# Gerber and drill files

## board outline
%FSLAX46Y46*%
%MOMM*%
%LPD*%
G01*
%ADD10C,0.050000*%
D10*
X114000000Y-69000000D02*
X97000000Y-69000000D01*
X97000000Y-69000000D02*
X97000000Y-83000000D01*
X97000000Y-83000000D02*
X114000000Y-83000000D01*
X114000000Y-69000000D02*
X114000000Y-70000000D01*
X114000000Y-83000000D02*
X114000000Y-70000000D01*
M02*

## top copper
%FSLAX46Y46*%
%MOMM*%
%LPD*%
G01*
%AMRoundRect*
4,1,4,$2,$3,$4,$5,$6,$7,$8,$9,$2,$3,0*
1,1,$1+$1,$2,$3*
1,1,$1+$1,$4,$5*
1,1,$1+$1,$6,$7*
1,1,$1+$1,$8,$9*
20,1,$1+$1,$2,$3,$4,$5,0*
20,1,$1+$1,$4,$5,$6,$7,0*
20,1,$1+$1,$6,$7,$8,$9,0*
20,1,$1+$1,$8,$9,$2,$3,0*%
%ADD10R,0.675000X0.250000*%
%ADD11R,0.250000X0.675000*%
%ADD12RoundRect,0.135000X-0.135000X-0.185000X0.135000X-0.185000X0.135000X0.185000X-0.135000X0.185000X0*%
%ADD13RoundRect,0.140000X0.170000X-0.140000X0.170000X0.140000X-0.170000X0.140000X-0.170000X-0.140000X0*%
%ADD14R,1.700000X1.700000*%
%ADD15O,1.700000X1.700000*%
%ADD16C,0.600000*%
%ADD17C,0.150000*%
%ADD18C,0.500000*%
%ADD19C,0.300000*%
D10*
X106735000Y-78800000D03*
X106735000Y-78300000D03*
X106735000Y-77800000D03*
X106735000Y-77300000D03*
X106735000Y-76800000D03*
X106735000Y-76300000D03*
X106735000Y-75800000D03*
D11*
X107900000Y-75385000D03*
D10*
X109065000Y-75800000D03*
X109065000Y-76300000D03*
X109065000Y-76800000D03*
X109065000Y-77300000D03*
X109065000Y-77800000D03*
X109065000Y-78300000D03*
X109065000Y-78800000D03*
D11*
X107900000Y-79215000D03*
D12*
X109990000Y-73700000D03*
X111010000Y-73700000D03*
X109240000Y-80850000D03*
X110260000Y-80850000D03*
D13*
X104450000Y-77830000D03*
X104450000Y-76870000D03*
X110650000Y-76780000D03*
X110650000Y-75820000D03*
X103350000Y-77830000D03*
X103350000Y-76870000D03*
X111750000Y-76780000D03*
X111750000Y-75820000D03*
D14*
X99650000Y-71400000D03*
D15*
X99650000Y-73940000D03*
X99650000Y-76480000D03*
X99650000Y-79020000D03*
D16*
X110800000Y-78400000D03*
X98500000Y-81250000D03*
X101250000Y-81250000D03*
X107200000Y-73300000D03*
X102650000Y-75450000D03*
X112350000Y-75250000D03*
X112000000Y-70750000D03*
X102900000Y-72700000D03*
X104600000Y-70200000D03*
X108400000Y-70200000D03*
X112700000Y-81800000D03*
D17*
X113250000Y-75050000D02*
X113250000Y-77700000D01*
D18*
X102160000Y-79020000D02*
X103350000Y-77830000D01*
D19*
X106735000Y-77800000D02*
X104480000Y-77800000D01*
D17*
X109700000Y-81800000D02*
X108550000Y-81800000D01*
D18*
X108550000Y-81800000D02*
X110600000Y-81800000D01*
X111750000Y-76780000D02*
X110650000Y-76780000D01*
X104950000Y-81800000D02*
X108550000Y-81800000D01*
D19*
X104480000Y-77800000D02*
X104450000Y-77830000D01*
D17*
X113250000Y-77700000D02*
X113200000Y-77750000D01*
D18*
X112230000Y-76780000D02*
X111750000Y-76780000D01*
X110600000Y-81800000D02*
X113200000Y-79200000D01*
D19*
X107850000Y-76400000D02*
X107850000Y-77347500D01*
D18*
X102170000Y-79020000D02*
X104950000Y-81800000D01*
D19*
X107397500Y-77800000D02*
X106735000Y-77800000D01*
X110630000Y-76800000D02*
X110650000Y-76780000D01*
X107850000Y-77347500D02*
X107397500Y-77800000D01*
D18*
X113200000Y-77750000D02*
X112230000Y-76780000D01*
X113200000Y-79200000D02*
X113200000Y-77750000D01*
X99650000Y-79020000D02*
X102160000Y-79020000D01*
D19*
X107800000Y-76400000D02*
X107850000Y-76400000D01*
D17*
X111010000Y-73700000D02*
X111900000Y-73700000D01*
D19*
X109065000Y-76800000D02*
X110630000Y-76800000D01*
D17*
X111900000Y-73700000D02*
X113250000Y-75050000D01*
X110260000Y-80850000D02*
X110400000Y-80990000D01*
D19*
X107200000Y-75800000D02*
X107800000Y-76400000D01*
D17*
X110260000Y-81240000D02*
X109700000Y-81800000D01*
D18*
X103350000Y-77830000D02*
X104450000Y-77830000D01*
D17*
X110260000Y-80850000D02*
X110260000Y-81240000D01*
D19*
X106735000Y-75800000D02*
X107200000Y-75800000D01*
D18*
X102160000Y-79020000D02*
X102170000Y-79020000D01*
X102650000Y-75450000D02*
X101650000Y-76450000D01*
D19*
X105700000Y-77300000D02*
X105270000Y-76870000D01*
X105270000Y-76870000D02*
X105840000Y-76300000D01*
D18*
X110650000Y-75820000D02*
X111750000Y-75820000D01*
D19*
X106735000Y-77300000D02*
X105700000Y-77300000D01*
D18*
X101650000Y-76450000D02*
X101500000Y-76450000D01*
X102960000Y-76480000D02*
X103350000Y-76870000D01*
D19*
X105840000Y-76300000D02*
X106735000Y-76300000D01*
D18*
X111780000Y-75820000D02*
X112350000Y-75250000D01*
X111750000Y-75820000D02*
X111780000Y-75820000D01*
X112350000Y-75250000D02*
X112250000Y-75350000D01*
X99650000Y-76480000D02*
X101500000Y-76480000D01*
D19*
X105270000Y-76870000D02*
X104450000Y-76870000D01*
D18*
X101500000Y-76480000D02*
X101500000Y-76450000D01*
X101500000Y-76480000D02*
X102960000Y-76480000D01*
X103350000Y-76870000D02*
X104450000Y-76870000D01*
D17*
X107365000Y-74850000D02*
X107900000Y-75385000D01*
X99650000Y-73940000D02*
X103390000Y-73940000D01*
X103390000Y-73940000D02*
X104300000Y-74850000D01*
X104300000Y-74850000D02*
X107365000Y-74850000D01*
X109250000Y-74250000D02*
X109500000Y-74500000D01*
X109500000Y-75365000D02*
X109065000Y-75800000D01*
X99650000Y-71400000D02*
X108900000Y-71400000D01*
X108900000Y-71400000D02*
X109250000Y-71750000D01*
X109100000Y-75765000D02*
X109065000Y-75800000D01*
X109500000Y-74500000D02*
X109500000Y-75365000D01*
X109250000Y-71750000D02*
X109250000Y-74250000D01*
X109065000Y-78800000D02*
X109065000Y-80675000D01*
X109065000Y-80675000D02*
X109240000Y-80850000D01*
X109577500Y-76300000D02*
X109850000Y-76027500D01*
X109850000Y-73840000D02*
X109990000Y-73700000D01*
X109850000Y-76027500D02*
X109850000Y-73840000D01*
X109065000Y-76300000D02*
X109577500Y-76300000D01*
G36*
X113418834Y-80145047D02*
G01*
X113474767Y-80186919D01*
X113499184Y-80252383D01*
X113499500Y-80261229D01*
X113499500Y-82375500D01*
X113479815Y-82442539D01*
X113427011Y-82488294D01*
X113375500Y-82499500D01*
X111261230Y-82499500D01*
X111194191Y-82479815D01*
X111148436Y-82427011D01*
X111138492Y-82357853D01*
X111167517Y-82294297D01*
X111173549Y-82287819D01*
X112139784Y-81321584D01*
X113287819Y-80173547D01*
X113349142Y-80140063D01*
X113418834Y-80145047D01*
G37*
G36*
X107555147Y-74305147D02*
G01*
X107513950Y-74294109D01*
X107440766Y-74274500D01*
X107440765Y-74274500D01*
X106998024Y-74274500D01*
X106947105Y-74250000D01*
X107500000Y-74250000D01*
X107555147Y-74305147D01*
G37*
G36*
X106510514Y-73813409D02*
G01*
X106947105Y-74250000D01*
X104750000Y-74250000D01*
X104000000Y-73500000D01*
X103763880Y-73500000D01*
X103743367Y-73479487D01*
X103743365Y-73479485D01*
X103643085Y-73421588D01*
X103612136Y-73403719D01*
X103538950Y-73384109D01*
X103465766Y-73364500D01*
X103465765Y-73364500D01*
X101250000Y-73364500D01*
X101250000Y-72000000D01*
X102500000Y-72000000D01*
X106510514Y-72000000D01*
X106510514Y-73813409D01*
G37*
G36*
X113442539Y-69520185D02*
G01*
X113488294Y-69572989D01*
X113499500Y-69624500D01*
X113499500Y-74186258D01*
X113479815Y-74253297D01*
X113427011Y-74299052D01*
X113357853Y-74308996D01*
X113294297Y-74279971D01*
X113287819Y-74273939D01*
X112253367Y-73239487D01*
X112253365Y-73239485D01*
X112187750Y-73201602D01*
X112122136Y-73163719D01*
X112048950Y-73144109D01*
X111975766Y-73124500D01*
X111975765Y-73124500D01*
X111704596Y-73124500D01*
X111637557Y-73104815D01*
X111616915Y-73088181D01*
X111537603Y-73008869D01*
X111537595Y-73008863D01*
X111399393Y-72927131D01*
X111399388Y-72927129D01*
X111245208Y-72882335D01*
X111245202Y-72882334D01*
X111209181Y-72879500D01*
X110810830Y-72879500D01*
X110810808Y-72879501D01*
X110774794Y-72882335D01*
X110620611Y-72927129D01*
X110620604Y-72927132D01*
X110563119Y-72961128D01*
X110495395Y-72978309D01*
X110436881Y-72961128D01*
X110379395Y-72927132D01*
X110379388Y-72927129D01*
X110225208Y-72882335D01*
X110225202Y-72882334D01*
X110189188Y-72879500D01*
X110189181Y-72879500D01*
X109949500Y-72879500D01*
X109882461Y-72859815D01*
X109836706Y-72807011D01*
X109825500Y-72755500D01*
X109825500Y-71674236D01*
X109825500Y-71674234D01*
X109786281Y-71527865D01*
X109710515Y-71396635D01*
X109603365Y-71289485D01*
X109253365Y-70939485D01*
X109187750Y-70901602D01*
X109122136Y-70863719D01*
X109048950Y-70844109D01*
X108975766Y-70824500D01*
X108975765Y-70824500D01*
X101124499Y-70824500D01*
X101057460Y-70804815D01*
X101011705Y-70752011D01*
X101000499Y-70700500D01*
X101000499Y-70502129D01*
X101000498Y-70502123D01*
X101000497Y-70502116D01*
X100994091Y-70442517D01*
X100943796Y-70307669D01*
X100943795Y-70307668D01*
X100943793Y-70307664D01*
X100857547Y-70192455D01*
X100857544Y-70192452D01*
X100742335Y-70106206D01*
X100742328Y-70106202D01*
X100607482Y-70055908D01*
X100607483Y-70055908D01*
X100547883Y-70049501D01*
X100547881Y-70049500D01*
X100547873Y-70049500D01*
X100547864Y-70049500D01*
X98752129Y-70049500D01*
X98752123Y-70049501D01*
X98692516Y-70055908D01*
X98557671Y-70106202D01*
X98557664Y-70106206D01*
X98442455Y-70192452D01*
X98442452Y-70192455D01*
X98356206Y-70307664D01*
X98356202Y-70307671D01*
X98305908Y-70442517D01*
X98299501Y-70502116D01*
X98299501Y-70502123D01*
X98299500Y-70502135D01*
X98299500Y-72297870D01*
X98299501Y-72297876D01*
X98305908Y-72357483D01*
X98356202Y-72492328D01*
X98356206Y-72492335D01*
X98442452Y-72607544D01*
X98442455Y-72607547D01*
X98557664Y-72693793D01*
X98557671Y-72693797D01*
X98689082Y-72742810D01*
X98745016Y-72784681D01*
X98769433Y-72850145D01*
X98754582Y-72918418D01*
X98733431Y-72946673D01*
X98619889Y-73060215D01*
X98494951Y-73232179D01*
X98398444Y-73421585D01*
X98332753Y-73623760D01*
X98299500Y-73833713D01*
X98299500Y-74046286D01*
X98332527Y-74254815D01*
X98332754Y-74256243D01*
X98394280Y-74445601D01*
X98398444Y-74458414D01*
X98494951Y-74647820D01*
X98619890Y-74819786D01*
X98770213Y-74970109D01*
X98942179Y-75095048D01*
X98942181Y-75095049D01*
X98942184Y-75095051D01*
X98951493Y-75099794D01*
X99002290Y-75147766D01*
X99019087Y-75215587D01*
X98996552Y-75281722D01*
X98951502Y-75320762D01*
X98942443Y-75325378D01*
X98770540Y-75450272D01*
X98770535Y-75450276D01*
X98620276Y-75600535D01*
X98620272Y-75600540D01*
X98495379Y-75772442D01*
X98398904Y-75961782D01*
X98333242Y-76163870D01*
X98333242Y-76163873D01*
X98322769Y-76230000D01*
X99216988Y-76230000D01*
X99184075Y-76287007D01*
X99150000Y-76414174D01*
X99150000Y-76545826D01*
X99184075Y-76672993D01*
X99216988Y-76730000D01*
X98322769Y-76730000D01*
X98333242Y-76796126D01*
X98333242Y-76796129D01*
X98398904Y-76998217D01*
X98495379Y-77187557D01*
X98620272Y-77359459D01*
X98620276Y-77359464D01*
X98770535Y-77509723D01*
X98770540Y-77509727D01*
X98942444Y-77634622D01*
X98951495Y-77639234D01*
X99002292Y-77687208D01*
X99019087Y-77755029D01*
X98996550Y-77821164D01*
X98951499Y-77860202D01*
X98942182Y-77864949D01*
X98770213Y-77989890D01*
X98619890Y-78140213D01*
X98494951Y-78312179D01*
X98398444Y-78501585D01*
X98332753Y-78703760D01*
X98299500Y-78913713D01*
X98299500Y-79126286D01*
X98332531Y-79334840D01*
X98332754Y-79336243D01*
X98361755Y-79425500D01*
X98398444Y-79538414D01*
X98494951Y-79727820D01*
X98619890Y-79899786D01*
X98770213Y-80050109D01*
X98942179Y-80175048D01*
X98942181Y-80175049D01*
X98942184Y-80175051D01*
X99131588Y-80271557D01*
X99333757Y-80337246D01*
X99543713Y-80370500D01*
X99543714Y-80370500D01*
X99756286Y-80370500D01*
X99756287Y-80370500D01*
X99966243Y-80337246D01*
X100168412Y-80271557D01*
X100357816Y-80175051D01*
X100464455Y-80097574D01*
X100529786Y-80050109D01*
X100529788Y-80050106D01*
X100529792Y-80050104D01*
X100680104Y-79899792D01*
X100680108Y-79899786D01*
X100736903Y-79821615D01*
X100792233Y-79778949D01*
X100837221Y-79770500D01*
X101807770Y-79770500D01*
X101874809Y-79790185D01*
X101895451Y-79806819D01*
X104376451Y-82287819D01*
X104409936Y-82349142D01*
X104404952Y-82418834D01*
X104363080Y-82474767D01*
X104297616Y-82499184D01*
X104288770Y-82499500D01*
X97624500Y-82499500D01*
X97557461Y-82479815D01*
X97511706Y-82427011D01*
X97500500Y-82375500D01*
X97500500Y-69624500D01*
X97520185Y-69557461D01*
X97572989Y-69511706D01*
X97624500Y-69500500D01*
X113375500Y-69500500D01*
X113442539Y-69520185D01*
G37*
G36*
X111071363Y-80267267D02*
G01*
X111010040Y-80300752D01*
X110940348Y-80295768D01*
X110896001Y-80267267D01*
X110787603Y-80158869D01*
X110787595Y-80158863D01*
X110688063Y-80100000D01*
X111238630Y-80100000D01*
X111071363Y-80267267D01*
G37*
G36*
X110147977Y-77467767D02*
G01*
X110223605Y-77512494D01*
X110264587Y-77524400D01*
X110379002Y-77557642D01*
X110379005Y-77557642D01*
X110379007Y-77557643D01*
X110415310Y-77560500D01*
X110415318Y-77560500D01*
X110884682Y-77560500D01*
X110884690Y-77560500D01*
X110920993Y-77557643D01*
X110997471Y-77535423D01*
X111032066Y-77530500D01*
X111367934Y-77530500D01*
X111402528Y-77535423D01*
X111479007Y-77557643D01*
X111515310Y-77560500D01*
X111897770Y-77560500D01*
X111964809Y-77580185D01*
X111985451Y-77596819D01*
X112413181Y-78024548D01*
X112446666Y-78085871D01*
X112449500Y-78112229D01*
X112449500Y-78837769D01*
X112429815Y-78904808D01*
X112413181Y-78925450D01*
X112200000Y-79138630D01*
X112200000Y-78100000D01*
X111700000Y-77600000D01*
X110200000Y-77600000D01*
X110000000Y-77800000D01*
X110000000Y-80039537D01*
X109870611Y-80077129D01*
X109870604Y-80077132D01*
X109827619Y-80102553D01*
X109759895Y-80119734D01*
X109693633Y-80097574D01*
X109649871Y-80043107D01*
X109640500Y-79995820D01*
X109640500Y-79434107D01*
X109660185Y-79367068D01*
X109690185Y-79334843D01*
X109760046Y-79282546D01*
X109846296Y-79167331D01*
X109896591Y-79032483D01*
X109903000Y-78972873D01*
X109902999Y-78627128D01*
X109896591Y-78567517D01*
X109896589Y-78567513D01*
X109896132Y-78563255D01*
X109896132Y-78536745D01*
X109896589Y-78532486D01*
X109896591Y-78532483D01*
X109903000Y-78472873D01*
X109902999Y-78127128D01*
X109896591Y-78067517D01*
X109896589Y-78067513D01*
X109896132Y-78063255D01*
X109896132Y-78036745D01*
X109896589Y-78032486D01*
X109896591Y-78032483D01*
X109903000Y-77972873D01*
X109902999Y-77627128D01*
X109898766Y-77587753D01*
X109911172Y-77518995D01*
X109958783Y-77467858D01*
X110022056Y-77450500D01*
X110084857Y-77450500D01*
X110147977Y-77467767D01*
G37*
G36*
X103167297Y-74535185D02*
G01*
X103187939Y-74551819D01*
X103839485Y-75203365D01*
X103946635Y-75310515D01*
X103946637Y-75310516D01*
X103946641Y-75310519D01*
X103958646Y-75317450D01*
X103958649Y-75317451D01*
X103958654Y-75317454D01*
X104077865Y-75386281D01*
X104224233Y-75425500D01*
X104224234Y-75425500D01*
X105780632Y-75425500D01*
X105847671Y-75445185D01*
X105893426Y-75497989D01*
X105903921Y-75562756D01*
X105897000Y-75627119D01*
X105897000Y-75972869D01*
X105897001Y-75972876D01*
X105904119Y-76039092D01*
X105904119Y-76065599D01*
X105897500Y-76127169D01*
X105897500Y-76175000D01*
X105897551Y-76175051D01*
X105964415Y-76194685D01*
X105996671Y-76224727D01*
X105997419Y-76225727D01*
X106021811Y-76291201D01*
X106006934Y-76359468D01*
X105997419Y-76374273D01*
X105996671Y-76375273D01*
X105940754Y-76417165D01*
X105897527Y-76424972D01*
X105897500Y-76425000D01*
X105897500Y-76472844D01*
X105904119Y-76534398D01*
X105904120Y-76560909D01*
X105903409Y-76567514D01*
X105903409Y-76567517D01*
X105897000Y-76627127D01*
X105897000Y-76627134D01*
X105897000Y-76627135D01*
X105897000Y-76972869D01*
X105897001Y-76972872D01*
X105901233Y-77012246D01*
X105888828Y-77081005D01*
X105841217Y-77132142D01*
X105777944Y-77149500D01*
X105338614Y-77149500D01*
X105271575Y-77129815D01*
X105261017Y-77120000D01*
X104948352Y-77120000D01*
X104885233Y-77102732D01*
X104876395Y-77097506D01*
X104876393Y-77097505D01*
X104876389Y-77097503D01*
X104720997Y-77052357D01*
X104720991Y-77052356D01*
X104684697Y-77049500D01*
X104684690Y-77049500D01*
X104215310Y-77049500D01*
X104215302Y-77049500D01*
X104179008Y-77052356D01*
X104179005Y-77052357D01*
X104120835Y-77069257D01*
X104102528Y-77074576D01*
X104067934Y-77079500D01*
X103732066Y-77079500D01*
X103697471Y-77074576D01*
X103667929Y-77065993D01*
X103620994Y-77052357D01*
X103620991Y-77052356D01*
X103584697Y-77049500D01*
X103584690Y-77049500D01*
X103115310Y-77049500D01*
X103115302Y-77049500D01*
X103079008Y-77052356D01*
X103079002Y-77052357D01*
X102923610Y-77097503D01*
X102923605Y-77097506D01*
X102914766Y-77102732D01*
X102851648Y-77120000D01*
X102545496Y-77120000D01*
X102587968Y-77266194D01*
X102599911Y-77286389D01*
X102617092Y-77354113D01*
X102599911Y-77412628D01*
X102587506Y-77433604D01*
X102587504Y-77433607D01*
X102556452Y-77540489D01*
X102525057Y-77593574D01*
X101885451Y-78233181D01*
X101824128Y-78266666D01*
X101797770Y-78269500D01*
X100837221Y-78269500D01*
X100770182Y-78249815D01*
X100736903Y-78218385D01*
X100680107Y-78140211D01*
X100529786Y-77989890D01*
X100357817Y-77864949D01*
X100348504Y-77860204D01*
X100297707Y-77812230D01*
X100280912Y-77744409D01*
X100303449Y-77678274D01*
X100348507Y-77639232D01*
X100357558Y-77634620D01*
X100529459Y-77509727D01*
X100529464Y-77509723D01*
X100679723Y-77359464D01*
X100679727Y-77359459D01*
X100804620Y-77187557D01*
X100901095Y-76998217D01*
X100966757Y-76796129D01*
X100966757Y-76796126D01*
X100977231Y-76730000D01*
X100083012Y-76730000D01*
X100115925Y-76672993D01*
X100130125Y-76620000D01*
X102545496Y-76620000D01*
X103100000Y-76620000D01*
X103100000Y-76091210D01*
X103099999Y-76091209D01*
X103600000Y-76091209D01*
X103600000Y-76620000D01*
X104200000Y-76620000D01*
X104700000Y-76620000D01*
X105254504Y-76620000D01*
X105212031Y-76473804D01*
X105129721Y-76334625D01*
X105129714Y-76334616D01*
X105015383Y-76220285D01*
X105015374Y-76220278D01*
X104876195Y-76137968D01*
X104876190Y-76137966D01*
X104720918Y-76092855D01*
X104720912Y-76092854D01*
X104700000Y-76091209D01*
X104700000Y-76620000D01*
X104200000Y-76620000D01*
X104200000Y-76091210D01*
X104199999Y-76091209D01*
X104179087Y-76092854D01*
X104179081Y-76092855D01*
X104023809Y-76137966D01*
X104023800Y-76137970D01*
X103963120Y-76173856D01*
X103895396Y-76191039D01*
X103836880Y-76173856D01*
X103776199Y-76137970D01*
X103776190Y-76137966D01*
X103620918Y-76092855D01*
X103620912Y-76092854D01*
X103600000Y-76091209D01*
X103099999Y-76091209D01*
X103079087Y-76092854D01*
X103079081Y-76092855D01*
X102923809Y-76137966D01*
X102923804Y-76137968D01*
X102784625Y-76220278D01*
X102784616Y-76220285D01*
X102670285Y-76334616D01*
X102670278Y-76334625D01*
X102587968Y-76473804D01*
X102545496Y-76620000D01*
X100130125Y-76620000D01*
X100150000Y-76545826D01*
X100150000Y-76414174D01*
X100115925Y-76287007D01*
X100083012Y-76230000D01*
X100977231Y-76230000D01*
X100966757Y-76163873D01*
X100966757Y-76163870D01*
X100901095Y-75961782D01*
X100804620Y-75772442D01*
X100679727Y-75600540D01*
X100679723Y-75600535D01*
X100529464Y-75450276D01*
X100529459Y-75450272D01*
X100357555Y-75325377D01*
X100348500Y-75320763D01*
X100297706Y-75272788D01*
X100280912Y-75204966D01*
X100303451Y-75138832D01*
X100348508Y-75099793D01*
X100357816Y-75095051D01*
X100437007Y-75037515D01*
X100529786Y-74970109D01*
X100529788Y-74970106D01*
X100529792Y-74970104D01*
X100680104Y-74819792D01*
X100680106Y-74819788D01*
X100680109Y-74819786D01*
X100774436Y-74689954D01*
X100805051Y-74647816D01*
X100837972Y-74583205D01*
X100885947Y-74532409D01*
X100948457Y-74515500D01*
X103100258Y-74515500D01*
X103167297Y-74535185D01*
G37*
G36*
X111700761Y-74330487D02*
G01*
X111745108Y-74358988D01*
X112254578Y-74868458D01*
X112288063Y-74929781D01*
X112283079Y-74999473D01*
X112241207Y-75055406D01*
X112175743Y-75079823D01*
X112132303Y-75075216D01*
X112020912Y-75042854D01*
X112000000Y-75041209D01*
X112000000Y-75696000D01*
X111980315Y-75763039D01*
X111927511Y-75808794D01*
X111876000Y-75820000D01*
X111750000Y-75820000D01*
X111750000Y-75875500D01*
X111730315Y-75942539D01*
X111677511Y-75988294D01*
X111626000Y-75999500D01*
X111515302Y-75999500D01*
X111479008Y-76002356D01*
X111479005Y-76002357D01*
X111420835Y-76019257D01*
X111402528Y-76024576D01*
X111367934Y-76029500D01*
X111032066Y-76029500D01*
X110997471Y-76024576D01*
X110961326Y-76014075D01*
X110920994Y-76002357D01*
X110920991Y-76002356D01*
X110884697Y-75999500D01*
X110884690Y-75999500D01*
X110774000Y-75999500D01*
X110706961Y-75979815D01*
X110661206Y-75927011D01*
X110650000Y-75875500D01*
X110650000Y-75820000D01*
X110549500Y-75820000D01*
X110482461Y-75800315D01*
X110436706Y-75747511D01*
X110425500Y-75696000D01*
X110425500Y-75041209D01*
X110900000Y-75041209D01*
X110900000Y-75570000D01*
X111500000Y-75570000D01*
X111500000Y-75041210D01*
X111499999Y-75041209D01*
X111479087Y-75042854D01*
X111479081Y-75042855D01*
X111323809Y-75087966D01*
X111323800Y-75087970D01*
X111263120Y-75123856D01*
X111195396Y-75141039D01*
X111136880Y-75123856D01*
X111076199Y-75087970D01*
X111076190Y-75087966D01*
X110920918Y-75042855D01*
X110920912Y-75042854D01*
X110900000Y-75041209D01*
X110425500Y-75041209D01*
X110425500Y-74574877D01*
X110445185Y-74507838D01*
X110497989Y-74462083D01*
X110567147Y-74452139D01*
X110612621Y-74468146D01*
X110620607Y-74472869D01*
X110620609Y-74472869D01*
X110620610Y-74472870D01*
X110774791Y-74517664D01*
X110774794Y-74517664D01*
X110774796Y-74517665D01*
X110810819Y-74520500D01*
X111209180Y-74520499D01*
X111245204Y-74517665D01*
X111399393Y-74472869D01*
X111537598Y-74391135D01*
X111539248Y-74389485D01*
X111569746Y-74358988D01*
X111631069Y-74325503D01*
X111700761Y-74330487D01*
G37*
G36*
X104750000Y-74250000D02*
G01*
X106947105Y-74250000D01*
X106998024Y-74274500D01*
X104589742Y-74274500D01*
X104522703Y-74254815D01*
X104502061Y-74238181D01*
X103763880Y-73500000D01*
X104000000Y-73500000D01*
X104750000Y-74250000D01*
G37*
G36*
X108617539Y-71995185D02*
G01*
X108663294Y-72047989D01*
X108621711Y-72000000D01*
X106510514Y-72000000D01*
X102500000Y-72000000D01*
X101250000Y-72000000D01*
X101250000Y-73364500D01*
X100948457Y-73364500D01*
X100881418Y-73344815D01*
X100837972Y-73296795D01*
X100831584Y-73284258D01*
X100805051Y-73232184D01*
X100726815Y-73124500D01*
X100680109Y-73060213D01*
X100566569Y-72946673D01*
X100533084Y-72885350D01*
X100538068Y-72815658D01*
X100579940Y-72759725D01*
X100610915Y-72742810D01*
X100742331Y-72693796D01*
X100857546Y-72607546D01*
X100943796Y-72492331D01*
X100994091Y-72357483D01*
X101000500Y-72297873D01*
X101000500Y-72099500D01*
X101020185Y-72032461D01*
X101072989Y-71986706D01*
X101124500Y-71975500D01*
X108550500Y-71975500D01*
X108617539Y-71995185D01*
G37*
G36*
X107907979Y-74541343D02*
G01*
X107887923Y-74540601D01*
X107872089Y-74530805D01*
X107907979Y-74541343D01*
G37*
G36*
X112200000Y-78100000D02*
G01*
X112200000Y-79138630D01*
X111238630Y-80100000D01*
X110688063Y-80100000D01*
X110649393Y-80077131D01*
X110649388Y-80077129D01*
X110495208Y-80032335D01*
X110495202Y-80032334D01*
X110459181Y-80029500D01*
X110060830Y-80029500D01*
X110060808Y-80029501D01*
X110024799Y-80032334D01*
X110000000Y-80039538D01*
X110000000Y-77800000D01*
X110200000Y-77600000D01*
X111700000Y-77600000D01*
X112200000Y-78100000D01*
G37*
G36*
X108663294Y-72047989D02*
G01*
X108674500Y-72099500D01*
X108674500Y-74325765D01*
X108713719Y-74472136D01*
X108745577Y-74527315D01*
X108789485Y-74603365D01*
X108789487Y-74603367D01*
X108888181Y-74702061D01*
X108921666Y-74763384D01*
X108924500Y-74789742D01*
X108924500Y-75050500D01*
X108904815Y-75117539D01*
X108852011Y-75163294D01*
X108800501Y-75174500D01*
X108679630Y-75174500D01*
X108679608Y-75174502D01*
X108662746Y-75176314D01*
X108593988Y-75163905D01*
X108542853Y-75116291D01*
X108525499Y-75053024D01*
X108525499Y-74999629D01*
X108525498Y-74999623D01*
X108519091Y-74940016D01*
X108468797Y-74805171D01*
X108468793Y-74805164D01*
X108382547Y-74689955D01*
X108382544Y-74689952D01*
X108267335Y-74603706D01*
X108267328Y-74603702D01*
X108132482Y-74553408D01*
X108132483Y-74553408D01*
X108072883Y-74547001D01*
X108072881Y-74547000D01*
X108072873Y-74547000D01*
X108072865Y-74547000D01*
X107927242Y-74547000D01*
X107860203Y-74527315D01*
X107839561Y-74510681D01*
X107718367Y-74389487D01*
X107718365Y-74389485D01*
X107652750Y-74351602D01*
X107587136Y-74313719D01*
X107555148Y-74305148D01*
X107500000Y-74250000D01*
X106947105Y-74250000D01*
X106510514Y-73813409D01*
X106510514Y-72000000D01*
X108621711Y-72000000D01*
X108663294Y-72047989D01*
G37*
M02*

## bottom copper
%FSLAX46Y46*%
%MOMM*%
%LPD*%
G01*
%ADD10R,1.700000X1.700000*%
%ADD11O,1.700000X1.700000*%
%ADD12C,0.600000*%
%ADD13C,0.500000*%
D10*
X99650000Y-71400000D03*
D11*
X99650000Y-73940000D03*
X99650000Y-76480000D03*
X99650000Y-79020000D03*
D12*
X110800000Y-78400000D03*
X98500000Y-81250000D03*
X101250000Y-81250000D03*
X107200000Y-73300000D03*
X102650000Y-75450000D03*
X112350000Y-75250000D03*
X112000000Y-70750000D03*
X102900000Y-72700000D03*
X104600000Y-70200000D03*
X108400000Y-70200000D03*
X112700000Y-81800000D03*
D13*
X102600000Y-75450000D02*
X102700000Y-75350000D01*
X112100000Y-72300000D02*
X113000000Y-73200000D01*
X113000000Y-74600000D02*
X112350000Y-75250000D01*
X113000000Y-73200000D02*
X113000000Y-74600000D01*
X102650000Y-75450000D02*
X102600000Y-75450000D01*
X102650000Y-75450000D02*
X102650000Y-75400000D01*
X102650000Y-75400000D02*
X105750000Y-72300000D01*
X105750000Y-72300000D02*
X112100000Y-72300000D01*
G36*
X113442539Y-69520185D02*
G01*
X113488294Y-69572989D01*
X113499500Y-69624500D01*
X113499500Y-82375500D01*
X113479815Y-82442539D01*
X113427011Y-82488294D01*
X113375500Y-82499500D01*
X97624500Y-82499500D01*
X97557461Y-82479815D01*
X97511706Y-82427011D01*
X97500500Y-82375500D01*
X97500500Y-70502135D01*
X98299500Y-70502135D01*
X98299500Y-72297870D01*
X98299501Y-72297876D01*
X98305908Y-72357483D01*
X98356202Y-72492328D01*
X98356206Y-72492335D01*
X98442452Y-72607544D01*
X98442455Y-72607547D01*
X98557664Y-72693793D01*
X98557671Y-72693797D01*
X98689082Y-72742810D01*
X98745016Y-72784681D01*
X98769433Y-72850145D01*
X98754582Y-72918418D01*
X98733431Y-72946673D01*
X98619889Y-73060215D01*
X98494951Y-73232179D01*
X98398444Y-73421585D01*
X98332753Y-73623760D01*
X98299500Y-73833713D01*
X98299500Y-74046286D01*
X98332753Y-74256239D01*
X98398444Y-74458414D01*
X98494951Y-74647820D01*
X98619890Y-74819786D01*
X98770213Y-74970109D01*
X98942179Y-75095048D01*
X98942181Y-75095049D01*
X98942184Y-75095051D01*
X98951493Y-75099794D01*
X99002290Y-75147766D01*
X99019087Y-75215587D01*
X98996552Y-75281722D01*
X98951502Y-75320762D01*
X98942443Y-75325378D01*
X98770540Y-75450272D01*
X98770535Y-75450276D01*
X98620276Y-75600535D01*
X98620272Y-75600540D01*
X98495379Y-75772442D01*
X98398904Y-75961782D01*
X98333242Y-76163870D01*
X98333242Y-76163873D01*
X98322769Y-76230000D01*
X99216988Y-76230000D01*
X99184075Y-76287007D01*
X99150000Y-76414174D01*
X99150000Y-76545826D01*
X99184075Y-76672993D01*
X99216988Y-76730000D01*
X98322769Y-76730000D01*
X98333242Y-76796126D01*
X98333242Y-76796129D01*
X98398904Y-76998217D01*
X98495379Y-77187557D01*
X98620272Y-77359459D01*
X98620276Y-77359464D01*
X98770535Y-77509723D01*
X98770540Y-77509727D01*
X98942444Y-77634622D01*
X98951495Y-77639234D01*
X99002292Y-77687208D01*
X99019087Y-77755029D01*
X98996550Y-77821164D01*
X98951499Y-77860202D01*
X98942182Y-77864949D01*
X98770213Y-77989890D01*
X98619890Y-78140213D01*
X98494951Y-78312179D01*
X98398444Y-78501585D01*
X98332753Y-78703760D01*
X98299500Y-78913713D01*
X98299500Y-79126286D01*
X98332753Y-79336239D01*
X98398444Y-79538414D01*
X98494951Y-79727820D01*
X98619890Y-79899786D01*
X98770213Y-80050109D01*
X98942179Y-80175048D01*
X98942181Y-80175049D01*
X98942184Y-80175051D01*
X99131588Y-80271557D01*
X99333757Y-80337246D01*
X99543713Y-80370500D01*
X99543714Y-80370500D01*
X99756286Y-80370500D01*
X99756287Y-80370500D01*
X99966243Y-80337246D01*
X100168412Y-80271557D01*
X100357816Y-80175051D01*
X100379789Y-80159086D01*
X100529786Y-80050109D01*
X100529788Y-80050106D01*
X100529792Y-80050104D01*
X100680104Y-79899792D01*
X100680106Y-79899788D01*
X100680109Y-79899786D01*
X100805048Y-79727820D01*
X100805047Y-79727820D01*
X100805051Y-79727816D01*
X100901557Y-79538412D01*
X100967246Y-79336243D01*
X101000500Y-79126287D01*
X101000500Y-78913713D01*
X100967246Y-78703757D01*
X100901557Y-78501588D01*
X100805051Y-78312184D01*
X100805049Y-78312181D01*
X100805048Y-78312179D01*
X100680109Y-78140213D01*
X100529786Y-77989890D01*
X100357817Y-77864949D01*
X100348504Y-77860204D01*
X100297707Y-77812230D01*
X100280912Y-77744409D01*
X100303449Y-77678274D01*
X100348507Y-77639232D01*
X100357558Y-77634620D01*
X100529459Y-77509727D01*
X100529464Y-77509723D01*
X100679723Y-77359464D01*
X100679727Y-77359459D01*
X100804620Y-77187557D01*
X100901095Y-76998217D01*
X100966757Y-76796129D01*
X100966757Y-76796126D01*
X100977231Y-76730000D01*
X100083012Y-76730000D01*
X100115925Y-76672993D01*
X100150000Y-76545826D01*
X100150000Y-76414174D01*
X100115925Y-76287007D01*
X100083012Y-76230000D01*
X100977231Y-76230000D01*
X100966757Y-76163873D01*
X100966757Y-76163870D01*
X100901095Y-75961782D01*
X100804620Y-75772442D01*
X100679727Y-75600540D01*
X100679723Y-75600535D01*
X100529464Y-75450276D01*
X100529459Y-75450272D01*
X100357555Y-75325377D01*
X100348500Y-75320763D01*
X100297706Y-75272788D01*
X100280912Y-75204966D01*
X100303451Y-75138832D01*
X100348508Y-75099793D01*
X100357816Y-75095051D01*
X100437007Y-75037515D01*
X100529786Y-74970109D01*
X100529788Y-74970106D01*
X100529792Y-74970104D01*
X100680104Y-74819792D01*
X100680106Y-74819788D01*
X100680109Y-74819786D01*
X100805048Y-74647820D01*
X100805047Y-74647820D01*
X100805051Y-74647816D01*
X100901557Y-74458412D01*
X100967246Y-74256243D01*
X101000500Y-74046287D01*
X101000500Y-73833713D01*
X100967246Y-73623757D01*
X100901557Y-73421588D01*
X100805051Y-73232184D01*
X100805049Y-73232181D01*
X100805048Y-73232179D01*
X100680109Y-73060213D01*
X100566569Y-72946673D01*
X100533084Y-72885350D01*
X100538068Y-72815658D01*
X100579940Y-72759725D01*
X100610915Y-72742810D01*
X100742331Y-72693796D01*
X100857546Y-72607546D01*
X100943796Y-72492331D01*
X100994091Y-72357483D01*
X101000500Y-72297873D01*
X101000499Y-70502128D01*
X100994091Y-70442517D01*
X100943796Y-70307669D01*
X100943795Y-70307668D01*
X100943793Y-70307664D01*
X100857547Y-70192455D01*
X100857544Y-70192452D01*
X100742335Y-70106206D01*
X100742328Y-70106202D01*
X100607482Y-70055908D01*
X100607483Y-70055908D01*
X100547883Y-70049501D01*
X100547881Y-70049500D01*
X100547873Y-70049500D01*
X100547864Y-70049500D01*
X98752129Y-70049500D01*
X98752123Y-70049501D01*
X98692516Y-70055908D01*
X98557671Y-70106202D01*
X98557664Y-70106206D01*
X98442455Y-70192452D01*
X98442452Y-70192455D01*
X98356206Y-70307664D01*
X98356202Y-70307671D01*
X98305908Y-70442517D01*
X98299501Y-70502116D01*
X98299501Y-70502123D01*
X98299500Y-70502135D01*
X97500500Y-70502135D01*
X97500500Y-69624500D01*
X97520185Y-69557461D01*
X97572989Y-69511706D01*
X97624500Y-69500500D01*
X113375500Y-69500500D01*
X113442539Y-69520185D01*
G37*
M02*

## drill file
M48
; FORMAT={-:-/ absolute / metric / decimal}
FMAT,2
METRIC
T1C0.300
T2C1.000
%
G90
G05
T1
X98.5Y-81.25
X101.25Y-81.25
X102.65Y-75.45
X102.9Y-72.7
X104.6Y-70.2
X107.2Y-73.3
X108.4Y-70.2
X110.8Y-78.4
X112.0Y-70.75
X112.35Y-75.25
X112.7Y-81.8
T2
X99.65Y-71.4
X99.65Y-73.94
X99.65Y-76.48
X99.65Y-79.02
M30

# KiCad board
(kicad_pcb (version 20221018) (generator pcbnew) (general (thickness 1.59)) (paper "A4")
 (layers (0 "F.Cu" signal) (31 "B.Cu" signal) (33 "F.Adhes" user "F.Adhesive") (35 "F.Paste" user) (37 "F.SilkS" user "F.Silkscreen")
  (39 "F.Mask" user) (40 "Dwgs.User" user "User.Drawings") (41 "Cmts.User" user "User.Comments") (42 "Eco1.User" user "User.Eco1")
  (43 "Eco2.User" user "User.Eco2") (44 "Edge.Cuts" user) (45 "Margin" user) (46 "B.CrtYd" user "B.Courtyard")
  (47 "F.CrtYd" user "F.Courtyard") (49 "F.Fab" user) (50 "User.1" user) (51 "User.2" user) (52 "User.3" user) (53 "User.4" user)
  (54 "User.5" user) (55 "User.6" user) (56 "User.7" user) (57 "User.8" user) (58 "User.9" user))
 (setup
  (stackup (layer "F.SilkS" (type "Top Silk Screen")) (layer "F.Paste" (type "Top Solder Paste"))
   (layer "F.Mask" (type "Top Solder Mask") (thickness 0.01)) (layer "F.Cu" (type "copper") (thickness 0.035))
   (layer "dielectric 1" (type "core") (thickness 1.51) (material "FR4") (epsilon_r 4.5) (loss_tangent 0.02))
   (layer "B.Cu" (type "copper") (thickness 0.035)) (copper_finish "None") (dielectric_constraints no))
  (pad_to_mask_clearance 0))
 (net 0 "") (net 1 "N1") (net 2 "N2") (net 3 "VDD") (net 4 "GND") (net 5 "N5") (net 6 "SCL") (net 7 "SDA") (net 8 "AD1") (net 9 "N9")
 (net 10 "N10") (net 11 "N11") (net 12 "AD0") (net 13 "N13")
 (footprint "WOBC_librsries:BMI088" (layer "F.Cu") (at 107.9 77.3 90)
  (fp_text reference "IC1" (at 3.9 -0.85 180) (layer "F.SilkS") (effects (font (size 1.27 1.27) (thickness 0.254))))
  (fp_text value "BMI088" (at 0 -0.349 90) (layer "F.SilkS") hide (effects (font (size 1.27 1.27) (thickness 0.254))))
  (pad "1" smd rect (at -1.5 -1.165 90) (size 0.25 0.675) (layers "F.Cu" "F.Paste" "F.Mask") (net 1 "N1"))
  (pad "2" smd rect (at -1 -1.165 90) (size 0.25 0.675) (layers "F.Cu" "F.Paste" "F.Mask") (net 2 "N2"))
  (pad "3" smd rect (at -0.5 -1.165 90) (size 0.25 0.675) (layers "F.Cu" "F.Paste" "F.Mask") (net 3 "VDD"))
  (pad "4" smd rect (at 0 -1.165 90) (size 0.25 0.675) (layers "F.Cu" "F.Paste" "F.Mask") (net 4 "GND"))
  (pad "5" smd rect (at 0.5 -1.165 90) (size 0.25 0.675) (layers "F.Cu" "F.Paste" "F.Mask") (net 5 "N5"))
  (pad "6" smd rect (at 1 -1.165 90) (size 0.25 0.675) (layers "F.Cu" "F.Paste" "F.Mask") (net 4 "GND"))
  (pad "7" smd rect (at 1.5 -1.165 90) (size 0.25 0.675) (layers "F.Cu" "F.Paste" "F.Mask") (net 3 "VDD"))
  (pad "8" smd rect (at 1.915 0 180) (size 0.25 0.675) (layers "F.Cu" "F.Paste" "F.Mask") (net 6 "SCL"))
  (pad "9" smd rect (at 1.5 1.165 90) (size 0.25 0.675) (layers "F.Cu" "F.Paste" "F.Mask") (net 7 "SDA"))
  (pad "10" smd rect (at 1 1.165 90) (size 0.25 0.675) (layers "F.Cu" "F.Paste" "F.Mask") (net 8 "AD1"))
  (pad "11" smd rect (at 0.5 1.165 90) (size 0.25 0.675) (layers "F.Cu" "F.Paste" "F.Mask") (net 3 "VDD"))
  (pad "12" smd rect (at 0 1.165 90) (size 0.25 0.675) (layers "F.Cu" "F.Paste" "F.Mask") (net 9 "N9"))
  (pad "13" smd rect (at -0.5 1.165 90) (size 0.25 0.675) (layers "F.Cu" "F.Paste" "F.Mask") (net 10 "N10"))
  (pad "14" smd rect (at -1 1.165 90) (size 0.25 0.675) (layers "F.Cu" "F.Paste" "F.Mask") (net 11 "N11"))
  (pad "15" smd rect (at -1.5 1.165 90) (size 0.25 0.675) (layers "F.Cu" "F.Paste" "F.Mask") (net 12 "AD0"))
  (pad "16" smd rect (at -1.915 0 180) (size 0.25 0.675) (layers "F.Cu" "F.Paste" "F.Mask") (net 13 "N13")))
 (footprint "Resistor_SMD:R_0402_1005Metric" (layer "F.Cu") (at 110.5 73.7)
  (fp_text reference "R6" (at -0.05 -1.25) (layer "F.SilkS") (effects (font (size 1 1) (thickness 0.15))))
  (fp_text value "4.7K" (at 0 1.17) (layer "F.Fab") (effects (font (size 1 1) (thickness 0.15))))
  (pad "1" smd roundrect (at -0.51 0) (size 0.54 0.64) (layers "F.Cu" "F.Paste" "F.Mask") (roundrect_rratio 0.25) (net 8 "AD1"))
  (pad "2" smd roundrect (at 0.51 0) (size 0.54 0.64) (layers "F.Cu" "F.Paste" "F.Mask") (roundrect_rratio 0.25) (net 3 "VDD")))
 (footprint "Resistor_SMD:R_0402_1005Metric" (layer "F.Cu") (at 109.75 80.85)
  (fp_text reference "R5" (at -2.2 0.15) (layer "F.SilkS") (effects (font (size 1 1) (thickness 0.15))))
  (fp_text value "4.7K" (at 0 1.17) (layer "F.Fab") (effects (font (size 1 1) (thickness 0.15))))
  (pad "1" smd roundrect (at -0.51 0) (size 0.54 0.64) (layers "F.Cu" "F.Paste" "F.Mask") (roundrect_rratio 0.25) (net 12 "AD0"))
  (pad "2" smd roundrect (at 0.51 0) (size 0.54 0.64) (layers "F.Cu" "F.Paste" "F.Mask") (roundrect_rratio 0.25) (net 3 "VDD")))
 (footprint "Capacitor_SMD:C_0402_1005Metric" (layer "F.Cu") (at 104.45 77.35 90)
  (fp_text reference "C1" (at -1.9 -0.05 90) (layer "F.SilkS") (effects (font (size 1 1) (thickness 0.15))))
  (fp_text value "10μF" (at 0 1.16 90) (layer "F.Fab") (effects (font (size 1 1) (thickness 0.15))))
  (pad "1" smd roundrect (at -0.48 0 90) (size 0.56 0.62) (layers "F.Cu" "F.Paste" "F.Mask") (roundrect_rratio 0.25) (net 3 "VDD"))
  (pad "2" smd roundrect (at 0.48 0 90) (size 0.56 0.62) (layers "F.Cu" "F.Paste" "F.Mask") (roundrect_rratio 0.25) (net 4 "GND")))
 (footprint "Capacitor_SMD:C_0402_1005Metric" (layer "F.Cu") (at 110.65 76.3 90)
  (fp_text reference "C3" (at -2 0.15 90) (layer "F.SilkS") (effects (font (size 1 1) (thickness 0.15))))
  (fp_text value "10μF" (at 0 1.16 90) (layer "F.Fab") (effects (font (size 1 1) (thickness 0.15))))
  (pad "1" smd roundrect (at -0.48 0 90) (size 0.56 0.62) (layers "F.Cu" "F.Paste" "F.Mask") (roundrect_rratio 0.25) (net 3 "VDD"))
  (pad "2" smd roundrect (at 0.48 0 90) (size 0.56 0.62) (layers "F.Cu" "F.Paste" "F.Mask") (roundrect_rratio 0.25) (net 4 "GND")))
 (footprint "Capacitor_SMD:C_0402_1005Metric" (layer "F.Cu") (at 103.35 77.35 90)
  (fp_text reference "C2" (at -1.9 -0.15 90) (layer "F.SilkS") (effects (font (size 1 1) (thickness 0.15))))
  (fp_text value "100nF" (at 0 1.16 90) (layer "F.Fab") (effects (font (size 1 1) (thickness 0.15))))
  (pad "1" smd roundrect (at -0.48 0 90) (size 0.56 0.62) (layers "F.Cu" "F.Paste" "F.Mask") (roundrect_rratio 0.25) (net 3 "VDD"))
  (pad "2" smd roundrect (at 0.48 0 90) (size 0.56 0.62) (layers "F.Cu" "F.Paste" "F.Mask") (roundrect_rratio 0.25) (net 4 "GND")))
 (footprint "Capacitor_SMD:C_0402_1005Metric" (layer "F.Cu") (at 111.75 76.3 90)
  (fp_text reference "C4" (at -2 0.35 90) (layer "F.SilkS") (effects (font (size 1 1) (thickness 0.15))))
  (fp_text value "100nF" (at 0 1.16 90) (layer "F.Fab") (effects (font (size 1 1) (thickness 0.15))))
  (pad "1" smd roundrect (at -0.48 0 90) (size 0.56 0.62) (layers "F.Cu" "F.Paste" "F.Mask") (roundrect_rratio 0.25) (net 3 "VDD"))
  (pad "2" smd roundrect (at 0.48 0 90) (size 0.56 0.62) (layers "F.Cu" "F.Paste" "F.Mask") (roundrect_rratio 0.25) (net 4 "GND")))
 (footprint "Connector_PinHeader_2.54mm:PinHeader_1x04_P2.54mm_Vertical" (layer "F.Cu") (at 99.65 71.4)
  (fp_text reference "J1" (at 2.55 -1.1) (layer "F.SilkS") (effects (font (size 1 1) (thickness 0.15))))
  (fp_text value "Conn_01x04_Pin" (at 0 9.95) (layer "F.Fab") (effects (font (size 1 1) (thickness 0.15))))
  (pad "1" thru_hole rect (at 0 0) (size 1.7 1.7) (drill 1) (layers "*.Cu" "*.Mask") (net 7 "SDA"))
  (pad "2" thru_hole oval (at 0 2.54) (size 1.7 1.7) (drill 1) (layers "*.Cu" "*.Mask") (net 6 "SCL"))
  (pad "3" thru_hole oval (at 0 5.08) (size 1.7 1.7) (drill 1) (layers "*.Cu" "*.Mask") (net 4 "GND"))
  (pad "4" thru_hole oval (at 0 7.62) (size 1.7 1.7) (drill 1) (layers "*.Cu" "*.Mask") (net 3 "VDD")))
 (gr_line (start 114 69) (end 97 69) (stroke (width 0.05) (type default)) (layer "Edge.Cuts"))
 (gr_line (start 97 69) (end 97 83) (stroke (width 0.05) (type default)) (layer "Edge.Cuts"))
 (gr_line (start 97 83) (end 114 83) (stroke (width 0.05) (type default)) (layer "Edge.Cuts"))
 (gr_line (start 114 69) (end 114 70) (stroke (width 0.05) (type default)) (layer "Edge.Cuts"))
 (gr_line (start 114 83) (end 114 70) (stroke (width 0.05) (type default)) (layer "Edge.Cuts"))
 (segment (start 113.25 75.05) (end 113.25 77.7) (width 0.15) (layer "F.Cu") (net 3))
 (segment (start 102.16 79.02) (end 103.35 77.83) (width 0.5) (layer "F.Cu") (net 3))
 (segment (start 106.735 77.8) (end 104.48 77.8) (width 0.3) (layer "F.Cu") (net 3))
 (segment (start 109.7 81.8) (end 108.55 81.8) (width 0.15) (layer "F.Cu") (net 3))
 (segment (start 108.55 81.8) (end 110.6 81.8) (width 0.5) (layer "F.Cu") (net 3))
 (segment (start 111.75 76.78) (end 110.65 76.78) (width 0.5) (layer "F.Cu") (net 3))
 (segment (start 104.95 81.8) (end 108.55 81.8) (width 0.5) (layer "F.Cu") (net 3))
 (segment (start 104.48 77.8) (end 104.45 77.83) (width 0.3) (layer "F.Cu") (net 3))
 (segment (start 113.25 77.7) (end 113.2 77.75) (width 0.15) (layer "F.Cu") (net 3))
 (segment (start 112.23 76.78) (end 111.75 76.78) (width 0.5) (layer "F.Cu") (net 3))
 (segment (start 110.6 81.8) (end 113.2 79.2) (width 0.5) (layer "F.Cu") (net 3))
 (segment (start 107.85 76.4) (end 107.85 77.3475) (width 0.3) (layer "F.Cu") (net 3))
 (segment (start 102.17 79.02) (end 104.95 81.8) (width 0.5) (layer "F.Cu") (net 3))
 (segment (start 107.3975 77.8) (end 106.735 77.8) (width 0.3) (layer "F.Cu") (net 3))
 (segment (start 110.63 76.8) (end 110.65 76.78) (width 0.3) (layer "F.Cu") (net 3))
 (segment (start 107.85 77.3475) (end 107.3975 77.8) (width 0.3) (layer "F.Cu") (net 3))
 (segment (start 113.2 77.75) (end 112.23 76.78) (width 0.5) (layer "F.Cu") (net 3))
 (segment (start 113.2 79.2) (end 113.2 77.75) (width 0.5) (layer "F.Cu") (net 3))
 (segment (start 99.65 79.02) (end 102.16 79.02) (width 0.5) (layer "F.Cu") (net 3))
 (segment (start 107.8 76.4) (end 107.85 76.4) (width 0.3) (layer "F.Cu") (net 3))
 (segment (start 111.01 73.7) (end 111.9 73.7) (width 0.15) (layer "F.Cu") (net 3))
 (segment (start 109.065 76.8) (end 110.63 76.8) (width 0.3) (layer "F.Cu") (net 3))
 (segment (start 111.9 73.7) (end 113.25 75.05) (width 0.15) (layer "F.Cu") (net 3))
 (segment (start 110.26 80.85) (end 110.4 80.99) (width 0.15) (layer "F.Cu") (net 3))
 (segment (start 107.2 75.8) (end 107.8 76.4) (width 0.3) (layer "F.Cu") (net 3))
 (segment (start 110.26 81.24) (end 109.7 81.8) (width 0.15) (layer "F.Cu") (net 3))
 (segment (start 103.35 77.83) (end 104.45 77.83) (width 0.5) (layer "F.Cu") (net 3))
 (segment (start 110.26 80.85) (end 110.26 81.24) (width 0.15) (layer "F.Cu") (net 3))
 (segment (start 106.735 75.8) (end 107.2 75.8) (width 0.3) (layer "F.Cu") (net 3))
 (segment (start 102.16 79.02) (end 102.17 79.02) (width 0.5) (layer "F.Cu") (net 3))
 (segment (start 102.65 75.45) (end 101.65 76.45) (width 0.5) (layer "F.Cu") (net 4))
 (segment (start 105.7 77.3) (end 105.27 76.87) (width 0.3) (layer "F.Cu") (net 4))
 (segment (start 105.27 76.87) (end 105.84 76.3) (width 0.3) (layer "F.Cu") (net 4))
 (segment (start 110.65 75.82) (end 111.75 75.82) (width 0.5) (layer "F.Cu") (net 4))
 (segment (start 106.735 77.3) (end 105.7 77.3) (width 0.3) (layer "F.Cu") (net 4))
 (segment (start 101.65 76.45) (end 101.5 76.45) (width 0.5) (layer "F.Cu") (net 4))
 (segment (start 102.96 76.48) (end 103.35 76.87) (width 0.5) (layer "F.Cu") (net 4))
 (segment (start 105.84 76.3) (end 106.735 76.3) (width 0.3) (layer "F.Cu") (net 4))
 (segment (start 111.78 75.82) (end 112.35 75.25) (width 0.5) (layer "F.Cu") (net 4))
 (segment (start 111.75 75.82) (end 111.78 75.82) (width 0.5) (layer "F.Cu") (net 4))
 (segment (start 112.35 75.25) (end 112.25 75.35) (width 0.5) (layer "F.Cu") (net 4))
 (segment (start 99.65 76.48) (end 101.5 76.48) (width 0.5) (layer "F.Cu") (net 4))
 (segment (start 105.27 76.87) (end 104.45 76.87) (width 0.3) (layer "F.Cu") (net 4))
 (segment (start 101.5 76.48) (end 101.5 76.45) (width 0.5) (layer "F.Cu") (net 4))
 (segment (start 101.5 76.48) (end 102.96 76.48) (width 0.5) (layer "F.Cu") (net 4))
 (segment (start 103.35 76.87) (end 104.45 76.87) (width 0.5) (layer "F.Cu") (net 4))
 (via (at 110.8 78.4) (size 0.6) (drill 0.3) (layers "F.Cu" "B.Cu") (free) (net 4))
 (via (at 98.5 81.25) (size 0.6) (drill 0.3) (layers "F.Cu" "B.Cu") (free) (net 4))
 (via (at 101.25 81.25) (size 0.6) (drill 0.3) (layers "F.Cu" "B.Cu") (free) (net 4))
 (via (at 107.2 73.3) (size 0.6) (drill 0.3) (layers "F.Cu" "B.Cu") (free) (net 4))
 (via (at 102.65 75.45) (size 0.6) (drill 0.3) (layers "F.Cu" "B.Cu") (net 4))
 (via (at 112.35 75.25) (size 0.6) (drill 0.3) (layers "F.Cu" "B.Cu") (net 4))
 (via (at 112 70.75) (size 0.6) (drill 0.3) (layers "F.Cu" "B.Cu") (free) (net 4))
 (via (at 102.9 72.7) (size 0.6) (drill 0.3) (layers "F.Cu" "B.Cu") (free) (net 4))
 (via (at 104.6 70.2) (size 0.6) (drill 0.3) (layers "F.Cu" "B.Cu") (free) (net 4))
 (via (at 108.4 70.2) (size 0.6) (drill 0.3) (layers "F.Cu" "B.Cu") (free) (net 4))
 (via (at 112.7 81.8) (size 0.6) (drill 0.3) (layers "F.Cu" "B.Cu") (free) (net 4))
 (segment (start 102.6 75.45) (end 102.7 75.35) (width 0.5) (layer "B.Cu") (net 4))
 (segment (start 112.1 72.3) (end 113 73.2) (width 0.5) (layer "B.Cu") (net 4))
 (segment (start 113 74.6) (end 112.35 75.25) (width 0.5) (layer "B.Cu") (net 4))
 (segment (start 113 73.2) (end 113 74.6) (width 0.5) (layer "B.Cu") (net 4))
 (segment (start 102.65 75.45) (end 102.6 75.45) (width 0.5) (layer "B.Cu") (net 4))
 (segment (start 102.65 75.45) (end 102.65 75.4) (width 0.5) (layer "B.Cu") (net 4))
 (segment (start 102.65 75.4) (end 105.75 72.3) (width 0.5) (layer "B.Cu") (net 4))
 (segment (start 105.75 72.3) (end 112.1 72.3) (width 0.5) (layer "B.Cu") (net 4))
 (segment (start 107.365 74.85) (end 107.9 75.385) (width 0.15) (layer "F.Cu") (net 6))
 (segment (start 99.65 73.94) (end 103.39 73.94) (width 0.15) (layer "F.Cu") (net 6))
 (segment (start 103.39 73.94) (end 104.3 74.85) (width 0.15) (layer "F.Cu") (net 6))
 (segment (start 104.3 74.85) (end 107.365 74.85) (width 0.15) (layer "F.Cu") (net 6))
 (segment (start 109.25 74.25) (end 109.5 74.5) (width 0.15) (layer "F.Cu") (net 7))
 (segment (start 109.5 75.365) (end 109.065 75.8) (width 0.15) (layer "F.Cu") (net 7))
 (segment (start 99.65 71.4) (end 108.9 71.4) (width 0.15) (layer "F.Cu") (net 7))
 (segment (start 108.9 71.4) (end 109.25 71.75) (width 0.15) (layer "F.Cu") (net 7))
 (segment (start 109.1 75.765) (end 109.065 75.8) (width 0.15) (layer "F.Cu") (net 7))
 (segment (start 109.5 74.5) (end 109.5 75.365) (width 0.15) (layer "F.Cu") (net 7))
 (segment (start 109.25 71.75) (end 109.25 74.25) (width 0.15) (layer "F.Cu") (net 7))
 (segment (start 109.065 78.8) (end 109.065 80.675) (width 0.15) (layer "F.Cu") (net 12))
 (segment (start 109.065 80.675) (end 109.24 80.85) (width 0.15) (layer "F.Cu") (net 12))
 (segment (start 109.5775 76.3) (end 109.85 76.0275) (width 0.15) (layer "F.Cu") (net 8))
 (segment (start 109.85 73.84) (end 109.99 73.7) (width 0.15) (layer "F.Cu") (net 8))
 (segment (start 109.85 76.0275) (end 109.85 73.84) (width 0.15) (layer "F.Cu") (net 8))
 (segment (start 109.065 76.3) (end 109.5775 76.3) (width 0.15) (layer "F.Cu") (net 8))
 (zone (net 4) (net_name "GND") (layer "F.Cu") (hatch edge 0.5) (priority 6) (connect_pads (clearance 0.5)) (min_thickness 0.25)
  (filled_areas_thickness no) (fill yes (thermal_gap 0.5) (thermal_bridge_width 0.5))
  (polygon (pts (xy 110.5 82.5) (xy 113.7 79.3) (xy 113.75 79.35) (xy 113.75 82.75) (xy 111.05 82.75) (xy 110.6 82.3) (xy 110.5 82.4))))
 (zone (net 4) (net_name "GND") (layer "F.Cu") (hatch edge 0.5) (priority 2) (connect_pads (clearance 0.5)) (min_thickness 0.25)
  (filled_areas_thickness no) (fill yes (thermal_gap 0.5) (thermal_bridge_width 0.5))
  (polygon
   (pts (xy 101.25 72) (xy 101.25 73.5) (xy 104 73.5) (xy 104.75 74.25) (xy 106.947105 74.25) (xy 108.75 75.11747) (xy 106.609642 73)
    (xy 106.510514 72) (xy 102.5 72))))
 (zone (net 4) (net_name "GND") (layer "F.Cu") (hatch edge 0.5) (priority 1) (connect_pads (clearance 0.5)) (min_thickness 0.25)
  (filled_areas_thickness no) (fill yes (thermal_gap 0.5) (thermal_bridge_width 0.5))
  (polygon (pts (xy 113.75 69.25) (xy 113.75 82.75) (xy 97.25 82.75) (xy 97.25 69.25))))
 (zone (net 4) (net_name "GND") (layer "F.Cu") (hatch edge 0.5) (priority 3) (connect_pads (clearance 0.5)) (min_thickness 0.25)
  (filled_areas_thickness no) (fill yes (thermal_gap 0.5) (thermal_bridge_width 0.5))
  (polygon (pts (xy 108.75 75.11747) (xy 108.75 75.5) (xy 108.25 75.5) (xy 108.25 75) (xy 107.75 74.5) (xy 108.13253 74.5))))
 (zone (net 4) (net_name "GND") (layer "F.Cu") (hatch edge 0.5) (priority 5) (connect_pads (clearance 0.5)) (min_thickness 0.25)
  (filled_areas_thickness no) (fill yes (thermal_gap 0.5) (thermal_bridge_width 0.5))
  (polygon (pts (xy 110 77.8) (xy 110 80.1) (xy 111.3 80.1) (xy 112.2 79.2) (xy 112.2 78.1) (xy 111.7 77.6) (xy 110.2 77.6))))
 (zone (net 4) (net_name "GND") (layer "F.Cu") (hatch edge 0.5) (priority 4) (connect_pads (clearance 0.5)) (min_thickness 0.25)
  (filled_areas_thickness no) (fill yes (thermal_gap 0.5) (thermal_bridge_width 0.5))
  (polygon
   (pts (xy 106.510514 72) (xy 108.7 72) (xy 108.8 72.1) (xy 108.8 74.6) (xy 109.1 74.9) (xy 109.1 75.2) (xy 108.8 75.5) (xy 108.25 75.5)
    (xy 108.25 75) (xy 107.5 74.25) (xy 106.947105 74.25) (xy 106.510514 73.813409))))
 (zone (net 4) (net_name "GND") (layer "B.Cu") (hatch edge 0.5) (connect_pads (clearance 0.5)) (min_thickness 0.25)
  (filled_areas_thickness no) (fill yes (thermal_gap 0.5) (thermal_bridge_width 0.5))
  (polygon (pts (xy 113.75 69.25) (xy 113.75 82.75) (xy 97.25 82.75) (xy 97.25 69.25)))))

